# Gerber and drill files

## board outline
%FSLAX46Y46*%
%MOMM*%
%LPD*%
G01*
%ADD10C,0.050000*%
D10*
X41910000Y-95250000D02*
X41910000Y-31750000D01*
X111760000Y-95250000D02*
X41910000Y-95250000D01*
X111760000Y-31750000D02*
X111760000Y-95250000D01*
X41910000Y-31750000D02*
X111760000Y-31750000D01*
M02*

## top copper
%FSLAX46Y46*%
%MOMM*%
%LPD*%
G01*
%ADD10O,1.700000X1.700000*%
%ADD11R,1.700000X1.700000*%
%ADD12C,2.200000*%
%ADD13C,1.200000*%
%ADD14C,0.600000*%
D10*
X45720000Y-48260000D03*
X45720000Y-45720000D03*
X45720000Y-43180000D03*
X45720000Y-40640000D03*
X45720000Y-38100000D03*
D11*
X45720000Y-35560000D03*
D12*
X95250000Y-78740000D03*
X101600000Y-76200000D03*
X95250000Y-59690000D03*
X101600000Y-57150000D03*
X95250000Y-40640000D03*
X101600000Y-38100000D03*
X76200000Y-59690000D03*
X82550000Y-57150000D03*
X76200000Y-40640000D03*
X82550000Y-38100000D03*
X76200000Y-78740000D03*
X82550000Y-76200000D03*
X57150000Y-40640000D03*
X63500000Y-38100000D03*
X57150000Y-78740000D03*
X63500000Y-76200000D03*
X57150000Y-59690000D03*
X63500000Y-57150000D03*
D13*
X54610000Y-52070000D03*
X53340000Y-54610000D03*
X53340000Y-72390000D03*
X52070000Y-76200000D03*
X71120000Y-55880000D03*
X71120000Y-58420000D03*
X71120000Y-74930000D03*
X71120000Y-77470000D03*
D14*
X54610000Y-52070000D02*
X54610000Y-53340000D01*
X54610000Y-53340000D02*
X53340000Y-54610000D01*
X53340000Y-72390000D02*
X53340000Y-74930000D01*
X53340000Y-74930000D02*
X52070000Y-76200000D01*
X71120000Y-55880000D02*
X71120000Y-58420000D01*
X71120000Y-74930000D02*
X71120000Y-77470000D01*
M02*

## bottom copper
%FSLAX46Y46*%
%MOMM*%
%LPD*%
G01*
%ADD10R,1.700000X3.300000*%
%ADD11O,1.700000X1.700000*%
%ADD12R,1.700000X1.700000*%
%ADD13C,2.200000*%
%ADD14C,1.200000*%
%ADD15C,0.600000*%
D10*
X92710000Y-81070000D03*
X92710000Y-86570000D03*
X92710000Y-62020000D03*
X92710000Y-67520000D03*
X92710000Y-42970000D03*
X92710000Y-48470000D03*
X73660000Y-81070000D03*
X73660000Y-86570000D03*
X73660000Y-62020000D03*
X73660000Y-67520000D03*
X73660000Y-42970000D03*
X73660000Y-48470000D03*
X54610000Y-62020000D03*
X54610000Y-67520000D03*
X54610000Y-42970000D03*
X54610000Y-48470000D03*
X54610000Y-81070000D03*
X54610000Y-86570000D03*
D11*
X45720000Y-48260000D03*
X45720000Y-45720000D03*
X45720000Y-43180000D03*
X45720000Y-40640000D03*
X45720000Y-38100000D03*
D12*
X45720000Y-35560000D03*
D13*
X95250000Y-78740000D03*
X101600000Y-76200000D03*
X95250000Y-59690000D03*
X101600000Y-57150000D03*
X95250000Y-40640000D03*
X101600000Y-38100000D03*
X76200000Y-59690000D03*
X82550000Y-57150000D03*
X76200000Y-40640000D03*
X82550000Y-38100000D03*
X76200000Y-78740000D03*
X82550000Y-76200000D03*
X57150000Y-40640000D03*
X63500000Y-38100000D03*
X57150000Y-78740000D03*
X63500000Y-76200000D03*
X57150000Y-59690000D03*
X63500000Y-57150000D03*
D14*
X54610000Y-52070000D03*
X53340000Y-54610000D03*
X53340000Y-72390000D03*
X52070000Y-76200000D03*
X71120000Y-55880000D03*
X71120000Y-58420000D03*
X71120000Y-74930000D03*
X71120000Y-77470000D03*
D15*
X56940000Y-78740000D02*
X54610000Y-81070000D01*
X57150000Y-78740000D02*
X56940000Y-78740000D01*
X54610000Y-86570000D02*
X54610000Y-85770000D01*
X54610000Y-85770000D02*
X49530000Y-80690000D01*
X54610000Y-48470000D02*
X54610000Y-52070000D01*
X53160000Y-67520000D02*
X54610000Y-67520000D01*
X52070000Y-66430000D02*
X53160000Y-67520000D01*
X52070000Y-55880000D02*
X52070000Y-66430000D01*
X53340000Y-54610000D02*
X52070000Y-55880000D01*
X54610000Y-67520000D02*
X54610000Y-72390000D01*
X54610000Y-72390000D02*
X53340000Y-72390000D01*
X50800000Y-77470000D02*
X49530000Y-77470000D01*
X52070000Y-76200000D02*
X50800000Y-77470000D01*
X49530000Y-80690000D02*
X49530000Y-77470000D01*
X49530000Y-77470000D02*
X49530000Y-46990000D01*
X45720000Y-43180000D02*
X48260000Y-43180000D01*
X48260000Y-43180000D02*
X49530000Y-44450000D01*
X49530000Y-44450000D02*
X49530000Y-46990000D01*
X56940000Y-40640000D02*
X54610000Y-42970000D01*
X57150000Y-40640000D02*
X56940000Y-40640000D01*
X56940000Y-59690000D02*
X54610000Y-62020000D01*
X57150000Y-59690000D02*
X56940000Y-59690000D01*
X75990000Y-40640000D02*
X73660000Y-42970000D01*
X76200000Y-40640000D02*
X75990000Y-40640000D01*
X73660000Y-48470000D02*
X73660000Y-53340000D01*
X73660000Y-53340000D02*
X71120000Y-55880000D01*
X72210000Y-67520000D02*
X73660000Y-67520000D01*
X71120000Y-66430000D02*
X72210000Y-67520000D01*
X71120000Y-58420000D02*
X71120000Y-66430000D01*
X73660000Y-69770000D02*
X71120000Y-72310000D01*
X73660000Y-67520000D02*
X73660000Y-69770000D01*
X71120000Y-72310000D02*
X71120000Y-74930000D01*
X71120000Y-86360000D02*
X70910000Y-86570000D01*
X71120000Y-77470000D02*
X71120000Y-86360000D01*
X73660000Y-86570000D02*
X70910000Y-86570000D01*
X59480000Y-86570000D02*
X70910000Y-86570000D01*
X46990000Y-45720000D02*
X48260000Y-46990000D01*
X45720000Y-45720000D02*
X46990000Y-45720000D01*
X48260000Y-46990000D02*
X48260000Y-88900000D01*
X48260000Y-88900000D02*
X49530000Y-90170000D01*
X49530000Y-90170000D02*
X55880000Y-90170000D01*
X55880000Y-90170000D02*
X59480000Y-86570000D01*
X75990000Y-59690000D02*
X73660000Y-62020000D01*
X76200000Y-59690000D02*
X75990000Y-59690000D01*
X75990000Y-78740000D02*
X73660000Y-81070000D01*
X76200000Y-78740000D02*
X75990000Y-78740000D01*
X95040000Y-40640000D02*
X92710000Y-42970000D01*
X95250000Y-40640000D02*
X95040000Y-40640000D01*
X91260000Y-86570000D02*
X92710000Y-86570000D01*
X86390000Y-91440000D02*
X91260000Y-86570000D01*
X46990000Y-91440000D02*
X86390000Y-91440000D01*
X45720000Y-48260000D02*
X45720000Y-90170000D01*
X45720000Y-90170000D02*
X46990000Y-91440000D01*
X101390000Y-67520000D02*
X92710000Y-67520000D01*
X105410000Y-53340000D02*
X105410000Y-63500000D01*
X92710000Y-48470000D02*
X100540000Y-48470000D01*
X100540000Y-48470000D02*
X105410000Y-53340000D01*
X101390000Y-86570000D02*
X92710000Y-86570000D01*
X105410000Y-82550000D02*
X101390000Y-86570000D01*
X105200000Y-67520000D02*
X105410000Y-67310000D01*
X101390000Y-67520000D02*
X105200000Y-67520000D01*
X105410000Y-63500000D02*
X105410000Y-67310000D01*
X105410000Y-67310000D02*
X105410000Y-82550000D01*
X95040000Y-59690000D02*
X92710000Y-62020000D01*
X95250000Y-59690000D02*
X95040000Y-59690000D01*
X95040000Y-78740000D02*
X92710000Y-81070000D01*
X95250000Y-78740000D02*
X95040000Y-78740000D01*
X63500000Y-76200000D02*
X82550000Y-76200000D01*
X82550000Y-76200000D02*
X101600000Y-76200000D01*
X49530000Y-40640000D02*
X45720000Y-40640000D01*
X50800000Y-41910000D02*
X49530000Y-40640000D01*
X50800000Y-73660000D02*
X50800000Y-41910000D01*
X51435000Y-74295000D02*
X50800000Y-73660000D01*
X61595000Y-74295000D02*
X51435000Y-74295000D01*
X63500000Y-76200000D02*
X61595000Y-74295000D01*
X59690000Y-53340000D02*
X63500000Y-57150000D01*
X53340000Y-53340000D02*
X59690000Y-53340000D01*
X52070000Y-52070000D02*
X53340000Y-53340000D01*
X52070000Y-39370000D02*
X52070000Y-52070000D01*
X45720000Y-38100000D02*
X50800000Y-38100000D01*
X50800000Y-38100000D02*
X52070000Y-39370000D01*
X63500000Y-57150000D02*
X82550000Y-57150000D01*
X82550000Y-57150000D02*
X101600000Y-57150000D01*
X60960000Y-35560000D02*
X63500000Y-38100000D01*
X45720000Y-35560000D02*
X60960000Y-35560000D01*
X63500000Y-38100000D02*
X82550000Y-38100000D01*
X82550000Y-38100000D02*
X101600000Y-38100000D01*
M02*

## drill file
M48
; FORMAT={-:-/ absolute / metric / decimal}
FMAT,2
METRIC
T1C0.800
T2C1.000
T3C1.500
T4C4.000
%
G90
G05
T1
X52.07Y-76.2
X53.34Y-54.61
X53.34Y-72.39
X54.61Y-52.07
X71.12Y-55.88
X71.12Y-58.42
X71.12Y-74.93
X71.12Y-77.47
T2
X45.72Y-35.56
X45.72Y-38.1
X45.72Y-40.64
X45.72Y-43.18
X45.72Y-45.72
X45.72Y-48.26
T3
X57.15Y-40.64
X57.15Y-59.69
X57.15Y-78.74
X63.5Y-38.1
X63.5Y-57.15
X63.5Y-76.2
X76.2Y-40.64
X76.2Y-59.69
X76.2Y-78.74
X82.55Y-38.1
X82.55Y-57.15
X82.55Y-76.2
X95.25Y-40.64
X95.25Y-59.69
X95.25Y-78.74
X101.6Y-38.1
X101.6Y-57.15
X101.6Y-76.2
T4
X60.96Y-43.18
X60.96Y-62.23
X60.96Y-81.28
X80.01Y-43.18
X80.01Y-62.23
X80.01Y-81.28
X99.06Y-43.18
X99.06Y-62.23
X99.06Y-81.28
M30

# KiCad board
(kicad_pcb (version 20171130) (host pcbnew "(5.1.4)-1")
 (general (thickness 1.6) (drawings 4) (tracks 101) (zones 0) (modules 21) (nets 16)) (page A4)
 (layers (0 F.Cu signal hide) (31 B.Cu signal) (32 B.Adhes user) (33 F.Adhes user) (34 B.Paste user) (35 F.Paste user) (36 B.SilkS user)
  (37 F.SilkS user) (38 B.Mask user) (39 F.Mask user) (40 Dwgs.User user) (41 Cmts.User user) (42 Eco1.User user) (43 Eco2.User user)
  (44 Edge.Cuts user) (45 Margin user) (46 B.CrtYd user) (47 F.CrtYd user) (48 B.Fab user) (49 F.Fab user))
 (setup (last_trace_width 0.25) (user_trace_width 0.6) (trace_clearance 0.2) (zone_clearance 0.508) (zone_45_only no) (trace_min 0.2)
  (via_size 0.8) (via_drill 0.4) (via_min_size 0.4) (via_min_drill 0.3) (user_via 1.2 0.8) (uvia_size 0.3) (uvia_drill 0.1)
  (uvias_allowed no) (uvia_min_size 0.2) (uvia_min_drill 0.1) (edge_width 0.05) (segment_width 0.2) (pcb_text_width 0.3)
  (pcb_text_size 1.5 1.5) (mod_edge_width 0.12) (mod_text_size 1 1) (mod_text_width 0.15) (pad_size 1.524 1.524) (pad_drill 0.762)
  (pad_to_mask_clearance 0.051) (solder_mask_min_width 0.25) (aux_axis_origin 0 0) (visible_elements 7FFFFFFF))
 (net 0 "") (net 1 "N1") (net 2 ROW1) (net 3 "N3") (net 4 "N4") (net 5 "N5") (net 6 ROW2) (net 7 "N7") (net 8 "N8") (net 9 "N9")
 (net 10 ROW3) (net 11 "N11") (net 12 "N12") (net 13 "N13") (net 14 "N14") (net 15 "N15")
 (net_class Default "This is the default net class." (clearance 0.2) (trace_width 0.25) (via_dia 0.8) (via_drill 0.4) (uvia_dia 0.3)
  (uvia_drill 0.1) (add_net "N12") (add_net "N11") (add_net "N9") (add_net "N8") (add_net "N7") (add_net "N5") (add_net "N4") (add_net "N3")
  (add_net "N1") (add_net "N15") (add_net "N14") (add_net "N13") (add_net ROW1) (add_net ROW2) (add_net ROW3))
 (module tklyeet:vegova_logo (layer F.Cu) (at 76.2 88.9)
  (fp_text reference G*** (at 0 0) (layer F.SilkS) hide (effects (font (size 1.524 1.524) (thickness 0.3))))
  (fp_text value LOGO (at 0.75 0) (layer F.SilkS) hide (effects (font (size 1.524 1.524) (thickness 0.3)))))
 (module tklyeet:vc (layer F.Cu) (at 96.52 89.535)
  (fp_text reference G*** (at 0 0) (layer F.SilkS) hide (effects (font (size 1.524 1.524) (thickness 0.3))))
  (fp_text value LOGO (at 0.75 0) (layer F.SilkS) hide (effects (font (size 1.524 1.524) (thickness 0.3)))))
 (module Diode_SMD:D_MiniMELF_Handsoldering (layer B.Cu) (at 92.71 83.82 90)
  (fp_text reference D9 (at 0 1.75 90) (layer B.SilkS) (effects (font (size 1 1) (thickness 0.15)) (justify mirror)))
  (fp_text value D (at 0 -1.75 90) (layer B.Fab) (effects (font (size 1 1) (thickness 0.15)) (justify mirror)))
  (pad 2 smd rect (at 2.75 0 90) (size 3.3 1.7) (layers B.Cu B.Paste B.Mask) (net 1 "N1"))
  (pad 1 smd rect (at -2.75 0 90) (size 3.3 1.7) (layers B.Cu B.Paste B.Mask) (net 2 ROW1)))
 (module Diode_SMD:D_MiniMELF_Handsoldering (layer B.Cu) (at 92.71 64.77 90)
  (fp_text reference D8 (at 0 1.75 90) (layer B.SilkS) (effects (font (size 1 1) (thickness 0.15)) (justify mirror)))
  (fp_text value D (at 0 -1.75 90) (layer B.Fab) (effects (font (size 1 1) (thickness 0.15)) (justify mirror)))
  (pad 2 smd rect (at 2.75 0 90) (size 3.3 1.7) (layers B.Cu B.Paste B.Mask) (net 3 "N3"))
  (pad 1 smd rect (at -2.75 0 90) (size 3.3 1.7) (layers B.Cu B.Paste B.Mask) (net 2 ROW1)))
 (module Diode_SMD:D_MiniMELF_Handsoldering (layer B.Cu) (at 92.71 45.72 90)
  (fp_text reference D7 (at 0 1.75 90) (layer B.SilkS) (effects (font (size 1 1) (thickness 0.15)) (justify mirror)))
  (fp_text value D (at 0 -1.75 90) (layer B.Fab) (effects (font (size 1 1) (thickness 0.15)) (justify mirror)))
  (pad 2 smd rect (at 2.75 0 90) (size 3.3 1.7) (layers B.Cu B.Paste B.Mask) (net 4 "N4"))
  (pad 1 smd rect (at -2.75 0 90) (size 3.3 1.7) (layers B.Cu B.Paste B.Mask) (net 2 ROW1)))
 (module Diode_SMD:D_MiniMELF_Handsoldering (layer B.Cu) (at 73.66 83.82 90)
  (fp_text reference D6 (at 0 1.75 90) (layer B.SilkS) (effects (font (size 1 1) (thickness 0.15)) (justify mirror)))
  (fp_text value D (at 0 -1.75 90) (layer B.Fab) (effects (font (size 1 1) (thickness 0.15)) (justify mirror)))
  (pad 2 smd rect (at 2.75 0 90) (size 3.3 1.7) (layers B.Cu B.Paste B.Mask) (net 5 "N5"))
  (pad 1 smd rect (at -2.75 0 90) (size 3.3 1.7) (layers B.Cu B.Paste B.Mask) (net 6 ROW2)))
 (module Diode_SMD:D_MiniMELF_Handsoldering (layer B.Cu) (at 73.66 64.77 90)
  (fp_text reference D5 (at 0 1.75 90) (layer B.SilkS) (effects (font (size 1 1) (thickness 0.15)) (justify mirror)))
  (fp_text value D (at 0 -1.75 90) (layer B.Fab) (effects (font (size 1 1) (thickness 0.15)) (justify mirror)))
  (pad 2 smd rect (at 2.75 0 90) (size 3.3 1.7) (layers B.Cu B.Paste B.Mask) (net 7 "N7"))
  (pad 1 smd rect (at -2.75 0 90) (size 3.3 1.7) (layers B.Cu B.Paste B.Mask) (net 6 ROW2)))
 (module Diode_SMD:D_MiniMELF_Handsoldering (layer B.Cu) (at 73.66 45.72 90)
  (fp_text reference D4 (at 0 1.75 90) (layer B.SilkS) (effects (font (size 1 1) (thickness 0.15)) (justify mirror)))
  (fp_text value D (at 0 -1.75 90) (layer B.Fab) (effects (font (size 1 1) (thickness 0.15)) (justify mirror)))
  (pad 2 smd rect (at 2.75 0 90) (size 3.3 1.7) (layers B.Cu B.Paste B.Mask) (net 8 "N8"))
  (pad 1 smd rect (at -2.75 0 90) (size 3.3 1.7) (layers B.Cu B.Paste B.Mask) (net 6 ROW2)))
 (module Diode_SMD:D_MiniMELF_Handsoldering (layer B.Cu) (at 54.61 64.77 90)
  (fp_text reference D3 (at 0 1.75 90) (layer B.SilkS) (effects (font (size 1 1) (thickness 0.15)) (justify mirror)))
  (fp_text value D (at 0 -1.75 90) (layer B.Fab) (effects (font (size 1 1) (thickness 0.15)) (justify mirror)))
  (pad 2 smd rect (at 2.75 0 90) (size 3.3 1.7) (layers B.Cu B.Paste B.Mask) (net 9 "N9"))
  (pad 1 smd rect (at -2.75 0 90) (size 3.3 1.7) (layers B.Cu B.Paste B.Mask) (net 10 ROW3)))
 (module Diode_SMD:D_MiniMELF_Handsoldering (layer B.Cu) (at 54.61 45.72 90)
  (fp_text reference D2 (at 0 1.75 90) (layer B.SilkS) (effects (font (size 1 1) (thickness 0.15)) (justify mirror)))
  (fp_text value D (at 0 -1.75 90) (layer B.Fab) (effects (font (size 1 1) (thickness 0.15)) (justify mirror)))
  (pad 2 smd rect (at 2.75 0 90) (size 3.3 1.7) (layers B.Cu B.Paste B.Mask) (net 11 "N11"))
  (pad 1 smd rect (at -2.75 0 90) (size 3.3 1.7) (layers B.Cu B.Paste B.Mask) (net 10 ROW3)))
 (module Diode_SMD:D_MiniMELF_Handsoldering (layer B.Cu) (at 54.61 83.82 90)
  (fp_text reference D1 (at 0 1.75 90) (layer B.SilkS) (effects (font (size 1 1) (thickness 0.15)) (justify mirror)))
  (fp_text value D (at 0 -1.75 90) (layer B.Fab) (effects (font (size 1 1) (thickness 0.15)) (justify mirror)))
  (pad 2 smd rect (at 2.75 0 90) (size 3.3 1.7) (layers B.Cu B.Paste B.Mask) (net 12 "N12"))
  (pad 1 smd rect (at -2.75 0 90) (size 3.3 1.7) (layers B.Cu B.Paste B.Mask) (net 10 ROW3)))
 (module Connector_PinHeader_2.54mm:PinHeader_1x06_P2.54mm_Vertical (layer F.Cu) (at 45.72 35.56)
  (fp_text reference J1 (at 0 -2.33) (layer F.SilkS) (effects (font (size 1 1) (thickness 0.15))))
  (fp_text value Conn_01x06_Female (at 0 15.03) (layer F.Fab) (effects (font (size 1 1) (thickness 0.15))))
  (pad 6 thru_hole oval (at 0 12.7) (size 1.7 1.7) (drill 1) (layers *.Cu *.Mask) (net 2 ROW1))
  (pad 5 thru_hole oval (at 0 10.16) (size 1.7 1.7) (drill 1) (layers *.Cu *.Mask) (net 6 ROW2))
  (pad 4 thru_hole oval (at 0 7.62) (size 1.7 1.7) (drill 1) (layers *.Cu *.Mask) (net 10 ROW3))
  (pad 3 thru_hole oval (at 0 5.08) (size 1.7 1.7) (drill 1) (layers *.Cu *.Mask) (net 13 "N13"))
  (pad 2 thru_hole oval (at 0 2.54) (size 1.7 1.7) (drill 1) (layers *.Cu *.Mask) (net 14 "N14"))
  (pad 1 thru_hole rect (at 0 0) (size 1.7 1.7) (drill 1) (layers *.Cu *.Mask) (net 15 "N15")))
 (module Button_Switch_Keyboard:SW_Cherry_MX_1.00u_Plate (layer F.Cu) (at 101.6 76.2)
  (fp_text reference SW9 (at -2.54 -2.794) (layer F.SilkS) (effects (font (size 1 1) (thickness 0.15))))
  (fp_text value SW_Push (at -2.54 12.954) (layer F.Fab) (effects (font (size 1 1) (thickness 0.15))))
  (pad "" np_thru_hole circle (at -2.54 5.08) (size 4 4) (drill 4) (layers *.Cu *.Mask))
  (pad 2 thru_hole circle (at -6.35 2.54) (size 2.2 2.2) (drill 1.5) (layers *.Cu *.Mask) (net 1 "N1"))
  (pad 1 thru_hole circle (at 0 0) (size 2.2 2.2) (drill 1.5) (layers *.Cu *.Mask) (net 13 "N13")))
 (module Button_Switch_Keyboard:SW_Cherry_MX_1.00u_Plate (layer F.Cu) (at 101.6 57.15)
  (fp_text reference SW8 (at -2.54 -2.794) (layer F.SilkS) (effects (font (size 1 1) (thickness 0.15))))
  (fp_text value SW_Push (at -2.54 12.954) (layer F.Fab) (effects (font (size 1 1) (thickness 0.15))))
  (pad "" np_thru_hole circle (at -2.54 5.08) (size 4 4) (drill 4) (layers *.Cu *.Mask))
  (pad 2 thru_hole circle (at -6.35 2.54) (size 2.2 2.2) (drill 1.5) (layers *.Cu *.Mask) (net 3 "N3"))
  (pad 1 thru_hole circle (at 0 0) (size 2.2 2.2) (drill 1.5) (layers *.Cu *.Mask) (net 14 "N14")))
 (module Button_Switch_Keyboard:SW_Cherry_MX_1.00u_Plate (layer F.Cu) (at 101.6 38.1)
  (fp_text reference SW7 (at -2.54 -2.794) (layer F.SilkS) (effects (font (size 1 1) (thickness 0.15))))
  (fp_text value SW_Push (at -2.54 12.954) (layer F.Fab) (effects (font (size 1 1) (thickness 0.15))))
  (pad "" np_thru_hole circle (at -2.54 5.08) (size 4 4) (drill 4) (layers *.Cu *.Mask))
  (pad 2 thru_hole circle (at -6.35 2.54) (size 2.2 2.2) (drill 1.5) (layers *.Cu *.Mask) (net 4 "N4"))
  (pad 1 thru_hole circle (at 0 0) (size 2.2 2.2) (drill 1.5) (layers *.Cu *.Mask) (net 15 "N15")))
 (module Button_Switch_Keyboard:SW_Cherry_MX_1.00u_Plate (layer F.Cu) (at 82.55 57.15)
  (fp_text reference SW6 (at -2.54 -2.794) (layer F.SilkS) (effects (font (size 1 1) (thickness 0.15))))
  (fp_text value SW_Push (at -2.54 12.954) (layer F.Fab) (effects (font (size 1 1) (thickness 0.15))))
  (pad "" np_thru_hole circle (at -2.54 5.08) (size 4 4) (drill 4) (layers *.Cu *.Mask))
  (pad 2 thru_hole circle (at -6.35 2.54) (size 2.2 2.2) (drill 1.5) (layers *.Cu *.Mask) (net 7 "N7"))
  (pad 1 thru_hole circle (at 0 0) (size 2.2 2.2) (drill 1.5) (layers *.Cu *.Mask) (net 14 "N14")))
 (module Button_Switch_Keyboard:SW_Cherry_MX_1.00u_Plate (layer F.Cu) (at 82.55 38.1)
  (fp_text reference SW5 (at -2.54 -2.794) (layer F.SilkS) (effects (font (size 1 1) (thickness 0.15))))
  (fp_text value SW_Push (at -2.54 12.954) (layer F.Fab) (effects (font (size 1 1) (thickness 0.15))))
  (pad "" np_thru_hole circle (at -2.54 5.08) (size 4 4) (drill 4) (layers *.Cu *.Mask))
  (pad 2 thru_hole circle (at -6.35 2.54) (size 2.2 2.2) (drill 1.5) (layers *.Cu *.Mask) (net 8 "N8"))
  (pad 1 thru_hole circle (at 0 0) (size 2.2 2.2) (drill 1.5) (layers *.Cu *.Mask) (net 15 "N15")))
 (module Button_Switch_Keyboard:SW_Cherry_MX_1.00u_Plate (layer F.Cu) (at 82.55 76.2)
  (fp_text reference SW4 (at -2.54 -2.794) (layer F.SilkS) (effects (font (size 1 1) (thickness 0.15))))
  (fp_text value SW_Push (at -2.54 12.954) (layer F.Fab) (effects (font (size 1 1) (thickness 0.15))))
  (pad "" np_thru_hole circle (at -2.54 5.08) (size 4 4) (drill 4) (layers *.Cu *.Mask))
  (pad 2 thru_hole circle (at -6.35 2.54) (size 2.2 2.2) (drill 1.5) (layers *.Cu *.Mask) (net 5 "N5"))
  (pad 1 thru_hole circle (at 0 0) (size 2.2 2.2) (drill 1.5) (layers *.Cu *.Mask) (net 13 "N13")))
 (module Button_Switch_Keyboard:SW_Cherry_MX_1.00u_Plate (layer F.Cu) (at 63.5 38.1)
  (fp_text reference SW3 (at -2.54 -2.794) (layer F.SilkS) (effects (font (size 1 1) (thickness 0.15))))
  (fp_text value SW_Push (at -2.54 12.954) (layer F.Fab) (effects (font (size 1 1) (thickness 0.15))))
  (pad "" np_thru_hole circle (at -2.54 5.08) (size 4 4) (drill 4) (layers *.Cu *.Mask))
  (pad 2 thru_hole circle (at -6.35 2.54) (size 2.2 2.2) (drill 1.5) (layers *.Cu *.Mask) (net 11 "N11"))
  (pad 1 thru_hole circle (at 0 0) (size 2.2 2.2) (drill 1.5) (layers *.Cu *.Mask) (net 15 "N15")))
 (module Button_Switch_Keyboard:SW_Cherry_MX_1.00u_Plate (layer F.Cu) (at 63.5 76.2)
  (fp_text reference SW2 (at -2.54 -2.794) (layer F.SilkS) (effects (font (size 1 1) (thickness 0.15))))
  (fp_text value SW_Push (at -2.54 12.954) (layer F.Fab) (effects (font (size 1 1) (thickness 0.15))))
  (pad "" np_thru_hole circle (at -2.54 5.08) (size 4 4) (drill 4) (layers *.Cu *.Mask))
  (pad 2 thru_hole circle (at -6.35 2.54) (size 2.2 2.2) (drill 1.5) (layers *.Cu *.Mask) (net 12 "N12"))
  (pad 1 thru_hole circle (at 0 0) (size 2.2 2.2) (drill 1.5) (layers *.Cu *.Mask) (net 13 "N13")))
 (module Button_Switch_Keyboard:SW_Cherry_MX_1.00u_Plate (layer F.Cu) (at 63.5 57.15)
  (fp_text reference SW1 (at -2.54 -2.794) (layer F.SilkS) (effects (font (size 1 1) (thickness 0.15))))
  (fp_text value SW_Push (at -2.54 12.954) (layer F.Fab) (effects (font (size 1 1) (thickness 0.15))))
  (pad "" np_thru_hole circle (at -2.54 5.08) (size 4 4) (drill 4) (layers *.Cu *.Mask))
  (pad 2 thru_hole circle (at -6.35 2.54) (size 2.2 2.2) (drill 1.5) (layers *.Cu *.Mask) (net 9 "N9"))
  (pad 1 thru_hole circle (at 0 0) (size 2.2 2.2) (drill 1.5) (layers *.Cu *.Mask) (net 14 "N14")))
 (gr_line (start 41.91 95.25) (end 41.91 31.75) (layer Edge.Cuts) (width 0.05))
 (gr_line (start 111.76 95.25) (end 41.91 95.25) (layer Edge.Cuts) (width 0.05))
 (gr_line (start 111.76 31.75) (end 111.76 95.25) (layer Edge.Cuts) (width 0.05))
 (gr_line (start 41.91 31.75) (end 111.76 31.75) (layer Edge.Cuts) (width 0.05))
 (segment (start 56.94 78.74) (end 54.61 81.07) (width 0.6) (layer B.Cu) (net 12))
 (segment (start 57.15 78.74) (end 56.94 78.74) (width 0.6) (layer B.Cu) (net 12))
 (segment (start 54.61 86.57) (end 54.61 85.77) (width 0.6) (layer B.Cu) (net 10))
 (segment (start 54.61 85.77) (end 49.53 80.69) (width 0.6) (layer B.Cu) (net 10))
 (segment (start 54.61 48.47) (end 54.61 52.07) (width 0.6) (layer B.Cu) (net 10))
 (via (at 54.61 52.07) (size 1.2) (drill 0.8) (layers F.Cu B.Cu) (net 10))
 (segment (start 54.61 52.07) (end 54.61 53.34) (width 0.6) (layer F.Cu) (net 10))
 (via (at 53.34 54.61) (size 1.2) (drill 0.8) (layers F.Cu B.Cu) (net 10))
 (segment (start 54.61 53.34) (end 53.34 54.61) (width 0.6) (layer F.Cu) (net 10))
 (segment (start 53.16 67.52) (end 54.61 67.52) (width 0.6) (layer B.Cu) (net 10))
 (segment (start 52.07 66.43) (end 53.16 67.52) (width 0.6) (layer B.Cu) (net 10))
 (segment (start 52.07 55.88) (end 52.07 66.43) (width 0.6) (layer B.Cu) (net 10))
 (segment (start 53.34 54.61) (end 52.07 55.88) (width 0.6) (layer B.Cu) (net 10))
 (segment (start 54.61 67.52) (end 54.61 72.39) (width 0.6) (layer B.Cu) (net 10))
 (segment (start 54.61 72.39) (end 53.34 72.39) (width 0.6) (layer B.Cu) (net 10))
 (via (at 53.34 72.39) (size 1.2) (drill 0.8) (layers F.Cu B.Cu) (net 10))
 (segment (start 53.34 72.39) (end 53.34 74.93) (width 0.6) (layer F.Cu) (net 10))
 (via (at 52.07 76.2) (size 1.2) (drill 0.8) (layers F.Cu B.Cu) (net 10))
 (segment (start 53.34 74.93) (end 52.07 76.2) (width 0.6) (layer F.Cu) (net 10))
 (segment (start 50.8 77.47) (end 49.53 77.47) (width 0.6) (layer B.Cu) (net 10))
 (segment (start 52.07 76.2) (end 50.8 77.47) (width 0.6) (layer B.Cu) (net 10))
 (segment (start 49.53 80.69) (end 49.53 77.47) (width 0.6) (layer B.Cu) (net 10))
 (segment (start 49.53 77.47) (end 49.53 46.99) (width 0.6) (layer B.Cu) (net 10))
 (segment (start 45.72 43.18) (end 48.26 43.18) (width 0.6) (layer B.Cu) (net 10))
 (segment (start 48.26 43.18) (end 49.53 44.45) (width 0.6) (layer B.Cu) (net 10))
 (segment (start 49.53 44.45) (end 49.53 46.99) (width 0.6) (layer B.Cu) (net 10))
 (segment (start 56.94 40.64) (end 54.61 42.97) (width 0.6) (layer B.Cu) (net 11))
 (segment (start 57.15 40.64) (end 56.94 40.64) (width 0.6) (layer B.Cu) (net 11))
 (segment (start 56.94 59.69) (end 54.61 62.02) (width 0.6) (layer B.Cu) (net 9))
 (segment (start 57.15 59.69) (end 56.94 59.69) (width 0.6) (layer B.Cu) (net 9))
 (segment (start 75.99 40.64) (end 73.66 42.97) (width 0.6) (layer B.Cu) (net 8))
 (segment (start 76.2 40.64) (end 75.99 40.64) (width 0.6) (layer B.Cu) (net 8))
 (via (at 71.12 55.88) (size 1.2) (drill 0.8) (layers F.Cu B.Cu) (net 6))
 (segment (start 73.66 48.47) (end 73.66 53.34) (width 0.6) (layer B.Cu) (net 6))
 (segment (start 73.66 53.34) (end 71.12 55.88) (width 0.6) (layer B.Cu) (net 6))
 (segment (start 71.12 55.88) (end 71.12 58.42) (width 0.6) (layer F.Cu) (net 6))
 (via (at 71.12 58.42) (size 1.2) (drill 0.8) (layers F.Cu B.Cu) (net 6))
 (segment (start 72.21 67.52) (end 73.66 67.52) (width 0.6) (layer B.Cu) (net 6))
 (segment (start 71.12 66.43) (end 72.21 67.52) (width 0.6) (layer B.Cu) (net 6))
 (segment (start 71.12 58.42) (end 71.12 66.43) (width 0.6) (layer B.Cu) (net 6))
 (segment (start 73.66 69.77) (end 71.12 72.31) (width 0.6) (layer B.Cu) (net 6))
 (segment (start 73.66 67.52) (end 73.66 69.77) (width 0.6) (layer B.Cu) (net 6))
 (via (at 71.12 74.93) (size 1.2) (drill 0.8) (layers F.Cu B.Cu) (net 6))
 (segment (start 71.12 72.31) (end 71.12 74.93) (width 0.6) (layer B.Cu) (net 6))
 (segment (start 71.12 74.93) (end 71.12 77.47) (width 0.6) (layer F.Cu) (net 6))
 (via (at 71.12 77.47) (size 1.2) (drill 0.8) (layers F.Cu B.Cu) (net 6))
 (segment (start 71.12 86.36) (end 70.91 86.57) (width 0.6) (layer B.Cu) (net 6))
 (segment (start 71.12 77.47) (end 71.12 86.36) (width 0.6) (layer B.Cu) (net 6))
 (segment (start 73.66 86.57) (end 70.91 86.57) (width 0.6) (layer B.Cu) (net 6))
 (segment (start 59.48 86.57) (end 70.91 86.57) (width 0.6) (layer B.Cu) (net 6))
 (segment (start 46.99 45.72) (end 48.26 46.99) (width 0.6) (layer B.Cu) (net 6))
 (segment (start 45.72 45.72) (end 46.99 45.72) (width 0.6) (layer B.Cu) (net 6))
 (segment (start 48.26 46.99) (end 48.26 88.9) (width 0.6) (layer B.Cu) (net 6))
 (segment (start 48.26 88.9) (end 49.53 90.17) (width 0.6) (layer B.Cu) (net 6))
 (segment (start 49.53 90.17) (end 55.88 90.17) (width 0.6) (layer B.Cu) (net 6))
 (segment (start 55.88 90.17) (end 59.48 86.57) (width 0.6) (layer B.Cu) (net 6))
 (segment (start 75.99 59.69) (end 73.66 62.02) (width 0.6) (layer B.Cu) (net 7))
 (segment (start 76.2 59.69) (end 75.99 59.69) (width 0.6) (layer B.Cu) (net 7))
 (segment (start 75.99 78.74) (end 73.66 81.07) (width 0.6) (layer B.Cu) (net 5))
 (segment (start 76.2 78.74) (end 75.99 78.74) (width 0.6) (layer B.Cu) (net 5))
 (segment (start 95.04 40.64) (end 92.71 42.97) (width 0.6) (layer B.Cu) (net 4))
 (segment (start 95.25 40.64) (end 95.04 40.64) (width 0.6) (layer B.Cu) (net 4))
 (segment (start 91.26 86.57) (end 92.71 86.57) (width 0.6) (layer B.Cu) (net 2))
 (segment (start 86.39 91.44) (end 91.26 86.57) (width 0.6) (layer B.Cu) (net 2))
 (segment (start 46.99 91.44) (end 86.39 91.44) (width 0.6) (layer B.Cu) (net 2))
 (segment (start 45.72 48.26) (end 45.72 90.17) (width 0.6) (layer B.Cu) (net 2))
 (segment (start 45.72 90.17) (end 46.99 91.44) (width 0.6) (layer B.Cu) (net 2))
 (segment (start 101.39 67.52) (end 92.71 67.52) (width 0.6) (layer B.Cu) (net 2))
 (segment (start 105.41 53.34) (end 105.41 63.5) (width 0.6) (layer B.Cu) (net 2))
 (segment (start 92.71 48.47) (end 100.54 48.47) (width 0.6) (layer B.Cu) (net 2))
 (segment (start 100.54 48.47) (end 105.41 53.34) (width 0.6) (layer B.Cu) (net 2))
 (segment (start 101.39 86.57) (end 92.71 86.57) (width 0.6) (layer B.Cu) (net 2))
 (segment (start 105.41 82.55) (end 101.39 86.57) (width 0.6) (layer B.Cu) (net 2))
 (segment (start 105.2 67.52) (end 105.41 67.31) (width 0.6) (layer B.Cu) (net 2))
 (segment (start 101.39 67.52) (end 105.2 67.52) (width 0.6) (layer B.Cu) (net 2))
 (segment (start 105.41 63.5) (end 105.41 67.31) (width 0.6) (layer B.Cu) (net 2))
 (segment (start 105.41 67.31) (end 105.41 82.55) (width 0.6) (layer B.Cu) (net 2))
 (segment (start 95.04 59.69) (end 92.71 62.02) (width 0.6) (layer B.Cu) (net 3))
 (segment (start 95.25 59.69) (end 95.04 59.69) (width 0.6) (layer B.Cu) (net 3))
 (segment (start 95.04 78.74) (end 92.71 81.07) (width 0.6) (layer B.Cu) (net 1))
 (segment (start 95.25 78.74) (end 95.04 78.74) (width 0.6) (layer B.Cu) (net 1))
 (segment (start 63.5 76.2) (end 82.55 76.2) (width 0.6) (layer B.Cu) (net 13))
 (segment (start 82.55 76.2) (end 101.6 76.2) (width 0.6) (layer B.Cu) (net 13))
 (segment (start 49.53 40.64) (end 45.72 40.64) (width 0.6) (layer B.Cu) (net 13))
 (segment (start 50.8 41.91) (end 49.53 40.64) (width 0.6) (layer B.Cu) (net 13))
 (segment (start 50.8 73.66) (end 50.8 41.91) (width 0.6) (layer B.Cu) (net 13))
 (segment (start 51.435 74.295) (end 50.8 73.66) (width 0.6) (layer B.Cu) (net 13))
 (segment (start 61.595 74.295) (end 51.435 74.295) (width 0.6) (layer B.Cu) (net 13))
 (segment (start 63.5 76.2) (end 61.595 74.295) (width 0.6) (layer B.Cu) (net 13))
 (segment (start 59.69 53.34) (end 63.5 57.15) (width 0.6) (layer B.Cu) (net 14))
 (segment (start 53.34 53.34) (end 59.69 53.34) (width 0.6) (layer B.Cu) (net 14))
 (segment (start 52.07 52.07) (end 53.34 53.34) (width 0.6) (layer B.Cu) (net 14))
 (segment (start 52.07 39.37) (end 52.07 52.07) (width 0.6) (layer B.Cu) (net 14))
 (segment (start 45.72 38.1) (end 50.8 38.1) (width 0.6) (layer B.Cu) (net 14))
 (segment (start 50.8 38.1) (end 52.07 39.37) (width 0.6) (layer B.Cu) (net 14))
 (segment (start 63.5 57.15) (end 82.55 57.15) (width 0.6) (layer B.Cu) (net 14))
 (segment (start 82.55 57.15) (end 101.6 57.15) (width 0.6) (layer B.Cu) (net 14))
 (segment (start 60.96 35.56) (end 63.5 38.1) (width 0.6) (layer B.Cu) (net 15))
 (segment (start 45.72 35.56) (end 60.96 35.56) (width 0.6) (layer B.Cu) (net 15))
 (segment (start 63.5 38.1) (end 82.55 38.1) (width 0.6) (layer B.Cu) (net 15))
 (segment (start 82.55 38.1) (end 101.6 38.1) (width 0.6) (layer B.Cu) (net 15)))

